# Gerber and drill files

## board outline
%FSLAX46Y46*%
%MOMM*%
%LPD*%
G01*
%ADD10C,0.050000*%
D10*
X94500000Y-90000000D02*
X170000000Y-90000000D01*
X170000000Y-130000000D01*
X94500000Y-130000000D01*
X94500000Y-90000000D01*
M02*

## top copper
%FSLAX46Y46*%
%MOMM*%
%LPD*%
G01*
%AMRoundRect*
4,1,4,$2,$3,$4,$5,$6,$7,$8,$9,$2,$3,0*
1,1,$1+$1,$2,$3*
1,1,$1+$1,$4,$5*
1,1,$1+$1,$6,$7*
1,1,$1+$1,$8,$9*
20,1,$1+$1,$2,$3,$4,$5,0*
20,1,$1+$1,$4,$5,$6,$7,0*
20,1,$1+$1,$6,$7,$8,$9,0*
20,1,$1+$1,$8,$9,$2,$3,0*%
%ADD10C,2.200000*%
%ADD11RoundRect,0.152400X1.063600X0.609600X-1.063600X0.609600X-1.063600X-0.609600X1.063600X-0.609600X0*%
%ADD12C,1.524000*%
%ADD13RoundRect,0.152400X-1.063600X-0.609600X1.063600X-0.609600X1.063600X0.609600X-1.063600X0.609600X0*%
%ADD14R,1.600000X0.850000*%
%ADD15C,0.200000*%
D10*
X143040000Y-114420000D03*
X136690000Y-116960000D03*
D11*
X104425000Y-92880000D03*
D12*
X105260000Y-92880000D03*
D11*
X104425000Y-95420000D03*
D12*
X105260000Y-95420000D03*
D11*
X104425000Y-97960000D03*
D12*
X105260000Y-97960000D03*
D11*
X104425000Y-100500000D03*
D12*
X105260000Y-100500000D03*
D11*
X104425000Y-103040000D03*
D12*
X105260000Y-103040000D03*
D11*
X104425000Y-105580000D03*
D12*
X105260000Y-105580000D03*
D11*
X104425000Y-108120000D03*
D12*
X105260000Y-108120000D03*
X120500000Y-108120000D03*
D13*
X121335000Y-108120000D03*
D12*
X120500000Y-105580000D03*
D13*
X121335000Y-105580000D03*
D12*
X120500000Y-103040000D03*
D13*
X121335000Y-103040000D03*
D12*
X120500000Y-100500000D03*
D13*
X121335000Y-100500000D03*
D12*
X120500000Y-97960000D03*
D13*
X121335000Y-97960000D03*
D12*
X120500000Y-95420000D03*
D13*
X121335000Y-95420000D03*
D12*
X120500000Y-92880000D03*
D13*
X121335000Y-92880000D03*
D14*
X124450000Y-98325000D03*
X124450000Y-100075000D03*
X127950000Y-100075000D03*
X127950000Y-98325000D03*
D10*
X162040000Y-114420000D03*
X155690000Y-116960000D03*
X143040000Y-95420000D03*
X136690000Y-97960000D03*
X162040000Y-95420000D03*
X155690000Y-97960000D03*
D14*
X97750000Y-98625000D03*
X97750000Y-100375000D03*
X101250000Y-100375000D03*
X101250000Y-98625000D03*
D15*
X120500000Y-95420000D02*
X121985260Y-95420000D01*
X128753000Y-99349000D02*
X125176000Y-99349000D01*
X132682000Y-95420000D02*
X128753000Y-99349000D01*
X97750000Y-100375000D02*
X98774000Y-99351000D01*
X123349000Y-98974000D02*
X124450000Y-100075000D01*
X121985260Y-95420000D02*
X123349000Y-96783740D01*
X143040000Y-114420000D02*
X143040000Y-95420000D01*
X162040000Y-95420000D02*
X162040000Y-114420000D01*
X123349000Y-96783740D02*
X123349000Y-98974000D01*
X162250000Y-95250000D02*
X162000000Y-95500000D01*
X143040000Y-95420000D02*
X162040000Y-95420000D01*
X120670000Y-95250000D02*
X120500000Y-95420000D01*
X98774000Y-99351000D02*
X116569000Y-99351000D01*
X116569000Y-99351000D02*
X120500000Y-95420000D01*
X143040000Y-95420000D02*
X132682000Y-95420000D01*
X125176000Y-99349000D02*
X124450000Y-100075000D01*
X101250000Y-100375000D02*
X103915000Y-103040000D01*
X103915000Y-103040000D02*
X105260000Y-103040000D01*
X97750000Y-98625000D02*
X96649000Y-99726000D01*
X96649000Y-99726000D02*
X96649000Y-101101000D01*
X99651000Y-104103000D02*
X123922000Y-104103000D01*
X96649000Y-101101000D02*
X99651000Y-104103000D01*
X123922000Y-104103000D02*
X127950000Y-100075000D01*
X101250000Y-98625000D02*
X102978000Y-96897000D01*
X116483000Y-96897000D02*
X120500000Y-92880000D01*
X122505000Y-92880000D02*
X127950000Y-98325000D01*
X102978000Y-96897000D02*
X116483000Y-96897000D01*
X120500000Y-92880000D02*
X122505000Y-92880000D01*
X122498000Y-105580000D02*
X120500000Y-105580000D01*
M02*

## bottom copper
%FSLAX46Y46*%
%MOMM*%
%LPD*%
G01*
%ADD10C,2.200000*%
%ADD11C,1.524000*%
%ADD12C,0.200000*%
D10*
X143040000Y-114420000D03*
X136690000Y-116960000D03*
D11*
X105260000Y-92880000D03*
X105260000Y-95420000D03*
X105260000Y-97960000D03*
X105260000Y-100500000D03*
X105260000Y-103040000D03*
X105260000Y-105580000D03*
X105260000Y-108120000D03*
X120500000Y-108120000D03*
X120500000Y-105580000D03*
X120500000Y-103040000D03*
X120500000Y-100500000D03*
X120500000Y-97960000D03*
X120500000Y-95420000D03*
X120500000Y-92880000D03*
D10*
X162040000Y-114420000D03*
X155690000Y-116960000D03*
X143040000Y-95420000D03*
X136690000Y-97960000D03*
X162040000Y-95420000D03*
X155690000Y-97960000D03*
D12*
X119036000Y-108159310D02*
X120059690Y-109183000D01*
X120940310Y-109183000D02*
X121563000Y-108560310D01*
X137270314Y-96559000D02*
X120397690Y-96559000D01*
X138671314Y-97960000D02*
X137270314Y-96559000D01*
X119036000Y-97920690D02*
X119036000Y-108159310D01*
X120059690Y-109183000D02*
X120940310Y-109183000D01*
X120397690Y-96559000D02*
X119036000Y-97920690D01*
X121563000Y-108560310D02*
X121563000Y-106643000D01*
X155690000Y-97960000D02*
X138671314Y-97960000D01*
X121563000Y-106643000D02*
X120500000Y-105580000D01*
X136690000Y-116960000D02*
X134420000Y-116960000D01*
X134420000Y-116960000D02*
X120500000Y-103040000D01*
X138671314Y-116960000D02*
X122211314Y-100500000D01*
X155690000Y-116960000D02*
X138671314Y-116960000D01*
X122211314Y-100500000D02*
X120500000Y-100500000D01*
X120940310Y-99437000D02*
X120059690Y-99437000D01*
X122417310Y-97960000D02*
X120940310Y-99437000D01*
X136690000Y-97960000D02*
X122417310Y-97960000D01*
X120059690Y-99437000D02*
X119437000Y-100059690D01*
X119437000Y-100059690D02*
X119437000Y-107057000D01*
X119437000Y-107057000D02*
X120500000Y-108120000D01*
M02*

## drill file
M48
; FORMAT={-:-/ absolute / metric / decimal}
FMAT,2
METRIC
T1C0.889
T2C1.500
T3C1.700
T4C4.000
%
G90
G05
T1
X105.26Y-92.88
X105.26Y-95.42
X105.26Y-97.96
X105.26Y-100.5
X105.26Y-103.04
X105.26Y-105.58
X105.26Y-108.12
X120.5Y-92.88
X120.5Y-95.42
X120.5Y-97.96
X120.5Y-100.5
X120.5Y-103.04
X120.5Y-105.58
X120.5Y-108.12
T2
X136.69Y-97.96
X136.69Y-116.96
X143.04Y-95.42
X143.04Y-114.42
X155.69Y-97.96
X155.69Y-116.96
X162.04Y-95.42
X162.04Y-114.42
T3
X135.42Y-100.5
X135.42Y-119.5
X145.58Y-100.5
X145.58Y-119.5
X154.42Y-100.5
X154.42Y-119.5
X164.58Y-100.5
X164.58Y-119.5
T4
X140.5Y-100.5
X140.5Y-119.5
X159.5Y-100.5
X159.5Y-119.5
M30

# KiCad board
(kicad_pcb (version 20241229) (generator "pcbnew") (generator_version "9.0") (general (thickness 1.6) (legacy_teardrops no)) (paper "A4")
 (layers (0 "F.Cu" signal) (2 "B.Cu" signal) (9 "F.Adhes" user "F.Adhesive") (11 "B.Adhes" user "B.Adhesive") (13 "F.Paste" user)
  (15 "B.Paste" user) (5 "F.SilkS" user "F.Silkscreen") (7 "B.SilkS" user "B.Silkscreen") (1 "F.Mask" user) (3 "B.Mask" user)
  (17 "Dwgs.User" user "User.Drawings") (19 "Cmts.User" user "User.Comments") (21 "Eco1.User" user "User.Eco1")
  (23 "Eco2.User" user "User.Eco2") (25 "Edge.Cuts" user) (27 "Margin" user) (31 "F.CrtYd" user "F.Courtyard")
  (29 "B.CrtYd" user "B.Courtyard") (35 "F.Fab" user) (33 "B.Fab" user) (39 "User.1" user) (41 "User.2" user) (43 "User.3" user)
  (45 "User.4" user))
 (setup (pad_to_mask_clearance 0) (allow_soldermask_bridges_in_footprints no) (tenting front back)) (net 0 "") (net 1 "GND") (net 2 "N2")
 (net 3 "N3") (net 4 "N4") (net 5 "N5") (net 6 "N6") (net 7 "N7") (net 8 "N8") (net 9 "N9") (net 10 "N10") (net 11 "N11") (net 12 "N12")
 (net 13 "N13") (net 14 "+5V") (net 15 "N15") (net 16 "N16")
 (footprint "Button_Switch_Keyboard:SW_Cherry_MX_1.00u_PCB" (layer "F.Cu") (at 143.04 114.42)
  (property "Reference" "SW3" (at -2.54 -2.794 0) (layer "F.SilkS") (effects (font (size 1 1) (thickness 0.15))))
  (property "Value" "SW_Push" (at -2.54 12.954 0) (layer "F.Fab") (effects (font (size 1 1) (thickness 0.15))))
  (pad "" np_thru_hole circle (at -7.62 5.08) (size 1.7 1.7) (drill 1.7) (layers "*.Cu" "*.Mask"))
  (pad "" np_thru_hole circle (at -2.54 5.08) (size 4 4) (drill 4) (layers "*.Cu" "*.Mask"))
  (pad "" np_thru_hole circle (at 2.54 5.08) (size 1.7 1.7) (drill 1.7) (layers "*.Cu" "*.Mask"))
  (pad "1" thru_hole circle (at 0 0) (size 2.2 2.2) (drill 1.5) (layers "*.Cu" "*.Mask") (remove_unused_layers no) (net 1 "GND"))
  (pad "2" thru_hole circle (at -6.35 2.54) (size 2.2 2.2) (drill 1.5) (layers "*.Cu" "*.Mask") (remove_unused_layers no) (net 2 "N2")))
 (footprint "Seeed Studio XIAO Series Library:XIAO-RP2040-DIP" (layer "F.Cu") (at 112.88 100.5)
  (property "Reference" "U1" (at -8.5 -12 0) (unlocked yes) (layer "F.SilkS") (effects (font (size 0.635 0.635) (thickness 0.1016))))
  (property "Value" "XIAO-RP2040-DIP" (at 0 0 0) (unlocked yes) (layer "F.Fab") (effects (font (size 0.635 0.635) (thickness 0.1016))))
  (pad "1" smd roundrect (at -8.455 -7.62 180) (size 2.432 1.524) (layers "F.Cu" "F.Mask") (roundrect_rratio 0.1) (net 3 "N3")
   (thermal_bridge_angle 45))
  (pad "1" thru_hole circle (at -7.62 -7.62 180) (size 1.524 1.524) (drill 0.889) (layers "*.Cu" "*.Mask") (remove_unused_layers no)
   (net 3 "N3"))
  (pad "2" smd roundrect (at -8.455 -5.08 180) (size 2.432 1.524) (layers "F.Cu" "F.Mask") (roundrect_rratio 0.1) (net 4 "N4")
   (thermal_bridge_angle 45))
  (pad "2" thru_hole circle (at -7.62 -5.08 180) (size 1.524 1.524) (drill 0.889) (layers "*.Cu" "*.Mask") (remove_unused_layers no)
   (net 4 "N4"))
  (pad "3" smd roundrect (at -8.455 -2.54 180) (size 2.432 1.524) (layers "F.Cu" "F.Mask") (roundrect_rratio 0.1) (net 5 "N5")
   (thermal_bridge_angle 45))
  (pad "3" thru_hole circle (at -7.62 -2.54 180) (size 1.524 1.524) (drill 0.889) (layers "*.Cu" "*.Mask") (remove_unused_layers no)
   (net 5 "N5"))
  (pad "4" smd roundrect (at -8.455 0 180) (size 2.432 1.524) (layers "F.Cu" "F.Mask") (roundrect_rratio 0.1) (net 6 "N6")
   (thermal_bridge_angle 45))
  (pad "4" thru_hole circle (at -7.62 0 180) (size 1.524 1.524) (drill 0.889) (layers "*.Cu" "*.Mask") (remove_unused_layers no)
   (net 6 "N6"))
  (pad "5" smd roundrect (at -8.455 2.54 180) (size 2.432 1.524) (layers "F.Cu" "F.Mask") (roundrect_rratio 0.1) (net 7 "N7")
   (thermal_bridge_angle 45))
  (pad "5" thru_hole circle (at -7.62 2.54 180) (size 1.524 1.524) (drill 0.889) (layers "*.Cu" "*.Mask") (remove_unused_layers no)
   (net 7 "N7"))
  (pad "6" smd roundrect (at -8.455 5.08 180) (size 2.432 1.524) (layers "F.Cu" "F.Mask") (roundrect_rratio 0.1) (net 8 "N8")
   (thermal_bridge_angle 45))
  (pad "6" thru_hole circle (at -7.62 5.08 180) (size 1.524 1.524) (drill 0.889) (layers "*.Cu" "*.Mask") (remove_unused_layers no)
   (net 8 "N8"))
  (pad "7" smd roundrect (at -8.455 7.62 180) (size 2.432 1.524) (layers "F.Cu" "F.Mask") (roundrect_rratio 0.1) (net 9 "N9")
   (thermal_bridge_angle 45))
  (pad "7" thru_hole circle (at -7.62 7.62 180) (size 1.524 1.524) (drill 0.889) (layers "*.Cu" "*.Mask") (remove_unused_layers no)
   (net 9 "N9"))
  (pad "8" thru_hole circle (at 7.62 7.62) (size 1.524 1.524) (drill 0.889) (layers "*.Cu" "*.Mask") (remove_unused_layers no)
   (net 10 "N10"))
  (pad "8" smd roundrect (at 8.455 7.62) (size 2.432 1.524) (layers "F.Cu" "F.Mask") (roundrect_rratio 0.1) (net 10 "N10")
   (thermal_bridge_angle 45))
  (pad "9" thru_hole circle (at 7.62 5.08) (size 1.524 1.524) (drill 0.889) (layers "*.Cu" "*.Mask") (remove_unused_layers no)
   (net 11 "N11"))
  (pad "9" smd roundrect (at 8.455 5.08) (size 2.432 1.524) (layers "F.Cu" "F.Mask") (roundrect_rratio 0.1) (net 11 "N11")
   (thermal_bridge_angle 45))
  (pad "10" thru_hole circle (at 7.62 2.54) (size 1.524 1.524) (drill 0.889) (layers "*.Cu" "*.Mask") (remove_unused_layers no) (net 2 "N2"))
  (pad "10" smd roundrect (at 8.455 2.54) (size 2.432 1.524) (layers "F.Cu" "F.Mask") (roundrect_rratio 0.1) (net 2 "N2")
   (thermal_bridge_angle 45))
  (pad "11" thru_hole circle (at 7.62 0) (size 1.524 1.524) (drill 0.889) (layers "*.Cu" "*.Mask") (remove_unused_layers no) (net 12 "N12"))
  (pad "11" smd roundrect (at 8.455 0) (size 2.432 1.524) (layers "F.Cu" "F.Mask") (roundrect_rratio 0.1) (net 12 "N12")
   (thermal_bridge_angle 45))
  (pad "12" thru_hole circle (at 7.62 -2.54) (size 1.524 1.524) (drill 0.889) (layers "*.Cu" "*.Mask") (remove_unused_layers no)
   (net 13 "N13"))
  (pad "12" smd roundrect (at 8.455 -2.54) (size 2.432 1.524) (layers "F.Cu" "F.Mask") (roundrect_rratio 0.1) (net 13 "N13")
   (thermal_bridge_angle 45))
  (pad "13" thru_hole circle (at 7.62 -5.08) (size 1.524 1.524) (drill 0.889) (layers "*.Cu" "*.Mask") (remove_unused_layers no)
   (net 1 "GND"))
  (pad "13" smd roundrect (at 8.455 -5.08) (size 2.432 1.524) (layers "F.Cu" "F.Mask") (roundrect_rratio 0.1) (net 1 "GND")
   (thermal_bridge_angle 45))
  (pad "14" thru_hole circle (at 7.62 -7.62) (size 1.524 1.524) (drill 0.889) (layers "*.Cu" "*.Mask") (remove_unused_layers no)
   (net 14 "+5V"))
  (pad "14" smd roundrect (at 8.455 -7.62) (size 2.432 1.524) (layers "F.Cu" "F.Mask") (roundrect_rratio 0.1) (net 14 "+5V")
   (thermal_bridge_angle 45)))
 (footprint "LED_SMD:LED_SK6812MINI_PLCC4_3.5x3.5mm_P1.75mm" (layer "F.Cu") (at 126.2 99.2)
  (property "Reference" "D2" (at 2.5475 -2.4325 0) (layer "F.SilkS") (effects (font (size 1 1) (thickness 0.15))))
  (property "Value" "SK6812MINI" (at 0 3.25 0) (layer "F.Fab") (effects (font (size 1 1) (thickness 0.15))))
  (pad "1" smd rect (at -1.75 -0.875) (size 1.6 0.85) (layers "F.Cu" "F.Mask" "F.Paste") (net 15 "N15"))
  (pad "2" smd rect (at -1.75 0.875) (size 1.6 0.85) (layers "F.Cu" "F.Mask" "F.Paste") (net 1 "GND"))
  (pad "3" smd rect (at 1.75 0.875) (size 1.6 0.85) (layers "F.Cu" "F.Mask" "F.Paste") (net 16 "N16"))
  (pad "4" smd rect (at 1.75 -0.875) (size 1.6 0.85) (layers "F.Cu" "F.Mask" "F.Paste") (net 14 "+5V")))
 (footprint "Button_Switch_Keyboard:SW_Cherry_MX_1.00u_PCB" (layer "F.Cu") (at 162.04 114.42)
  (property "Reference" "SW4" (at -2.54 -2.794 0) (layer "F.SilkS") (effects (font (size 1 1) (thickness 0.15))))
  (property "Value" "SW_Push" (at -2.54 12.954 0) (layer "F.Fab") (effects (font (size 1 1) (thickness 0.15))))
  (pad "" np_thru_hole circle (at -7.62 5.08) (size 1.7 1.7) (drill 1.7) (layers "*.Cu" "*.Mask"))
  (pad "" np_thru_hole circle (at -2.54 5.08) (size 4 4) (drill 4) (layers "*.Cu" "*.Mask"))
  (pad "" np_thru_hole circle (at 2.54 5.08) (size 1.7 1.7) (drill 1.7) (layers "*.Cu" "*.Mask"))
  (pad "1" thru_hole circle (at 0 0) (size 2.2 2.2) (drill 1.5) (layers "*.Cu" "*.Mask") (remove_unused_layers no) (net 1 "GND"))
  (pad "2" thru_hole circle (at -6.35 2.54) (size 2.2 2.2) (drill 1.5) (layers "*.Cu" "*.Mask") (remove_unused_layers no) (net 12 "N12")))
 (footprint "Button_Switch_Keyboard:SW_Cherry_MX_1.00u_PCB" (layer "F.Cu") (at 143.04 95.42)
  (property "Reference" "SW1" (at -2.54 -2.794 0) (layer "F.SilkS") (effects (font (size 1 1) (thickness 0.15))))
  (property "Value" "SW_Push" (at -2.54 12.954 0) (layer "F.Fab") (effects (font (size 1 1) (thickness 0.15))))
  (pad "" np_thru_hole circle (at -7.62 5.08) (size 1.7 1.7) (drill 1.7) (layers "*.Cu" "*.Mask"))
  (pad "" np_thru_hole circle (at -2.54 5.08) (size 4 4) (drill 4) (layers "*.Cu" "*.Mask"))
  (pad "" np_thru_hole circle (at 2.54 5.08) (size 1.7 1.7) (drill 1.7) (layers "*.Cu" "*.Mask"))
  (pad "1" thru_hole circle (at 0 0) (size 2.2 2.2) (drill 1.5) (layers "*.Cu" "*.Mask") (remove_unused_layers no) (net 1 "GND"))
  (pad "2" thru_hole circle (at -6.35 2.54) (size 2.2 2.2) (drill 1.5) (layers "*.Cu" "*.Mask") (remove_unused_layers no) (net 10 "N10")))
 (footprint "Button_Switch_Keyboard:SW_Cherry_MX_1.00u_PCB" (layer "F.Cu") (at 162.04 95.42)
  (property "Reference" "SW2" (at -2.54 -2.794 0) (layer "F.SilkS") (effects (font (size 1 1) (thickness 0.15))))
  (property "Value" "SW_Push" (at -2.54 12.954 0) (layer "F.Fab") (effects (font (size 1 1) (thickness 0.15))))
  (pad "" np_thru_hole circle (at -7.62 5.08) (size 1.7 1.7) (drill 1.7) (layers "*.Cu" "*.Mask"))
  (pad "" np_thru_hole circle (at -2.54 5.08) (size 4 4) (drill 4) (layers "*.Cu" "*.Mask"))
  (pad "" np_thru_hole circle (at 2.54 5.08) (size 1.7 1.7) (drill 1.7) (layers "*.Cu" "*.Mask"))
  (pad "1" thru_hole circle (at 0 0) (size 2.2 2.2) (drill 1.5) (layers "*.Cu" "*.Mask") (remove_unused_layers no) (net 1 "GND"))
  (pad "2" thru_hole circle (at -6.35 2.54) (size 2.2 2.2) (drill 1.5) (layers "*.Cu" "*.Mask") (remove_unused_layers no) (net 11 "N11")))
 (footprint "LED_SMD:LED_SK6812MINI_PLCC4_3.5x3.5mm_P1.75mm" (layer "F.Cu") (at 99.5 99.5)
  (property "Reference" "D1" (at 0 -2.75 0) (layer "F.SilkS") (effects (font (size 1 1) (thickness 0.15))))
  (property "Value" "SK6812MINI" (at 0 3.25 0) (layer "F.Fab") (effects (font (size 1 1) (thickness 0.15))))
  (pad "1" smd rect (at -1.75 -0.875) (size 1.6 0.85) (layers "F.Cu" "F.Mask" "F.Paste") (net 16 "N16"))
  (pad "2" smd rect (at -1.75 0.875) (size 1.6 0.85) (layers "F.Cu" "F.Mask" "F.Paste") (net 1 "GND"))
  (pad "3" smd rect (at 1.75 0.875) (size 1.6 0.85) (layers "F.Cu" "F.Mask" "F.Paste") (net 7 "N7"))
  (pad "4" smd rect (at 1.75 -0.875) (size 1.6 0.85) (layers "F.Cu" "F.Mask" "F.Paste") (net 14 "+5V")))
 (gr_rect (start 94.5 90) (end 170 130) (stroke (width 0.05) (type default)) (fill no) (layer "Edge.Cuts"))
 (segment (start 120.5 95.42) (end 121.98526 95.42) (width 0.2) (layer "F.Cu") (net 1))
 (segment (start 128.753 99.349) (end 125.176 99.349) (width 0.2) (layer "F.Cu") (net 1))
 (segment (start 132.682 95.42) (end 128.753 99.349) (width 0.2) (layer "F.Cu") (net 1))
 (segment (start 97.75 100.375) (end 98.774 99.351) (width 0.2) (layer "F.Cu") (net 1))
 (segment (start 123.349 98.974) (end 124.45 100.075) (width 0.2) (layer "F.Cu") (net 1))
 (segment (start 121.98526 95.42) (end 123.349 96.78374) (width 0.2) (layer "F.Cu") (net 1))
 (segment (start 143.04 114.42) (end 143.04 95.42) (width 0.2) (layer "F.Cu") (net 1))
 (segment (start 162.04 95.42) (end 162.04 114.42) (width 0.2) (layer "F.Cu") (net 1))
 (segment (start 123.349 96.78374) (end 123.349 98.974) (width 0.2) (layer "F.Cu") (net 1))
 (segment (start 162.25 95.25) (end 162 95.5) (width 0.2) (layer "F.Cu") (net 1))
 (segment (start 143.04 95.42) (end 162.04 95.42) (width 0.2) (layer "F.Cu") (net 1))
 (segment (start 120.67 95.25) (end 120.5 95.42) (width 0.2) (layer "F.Cu") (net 1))
 (segment (start 98.774 99.351) (end 116.569 99.351) (width 0.2) (layer "F.Cu") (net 1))
 (segment (start 116.569 99.351) (end 120.5 95.42) (width 0.2) (layer "F.Cu") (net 1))
 (segment (start 143.04 95.42) (end 132.682 95.42) (width 0.2) (layer "F.Cu") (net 1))
 (segment (start 125.176 99.349) (end 124.45 100.075) (width 0.2) (layer "F.Cu") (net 1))
 (segment (start 101.25 100.375) (end 103.915 103.04) (width 0.2) (layer "F.Cu") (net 7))
 (segment (start 103.915 103.04) (end 105.26 103.04) (width 0.2) (layer "F.Cu") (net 7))
 (segment (start 97.75 98.625) (end 96.649 99.726) (width 0.2) (layer "F.Cu") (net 16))
 (segment (start 96.649 99.726) (end 96.649 101.101) (width 0.2) (layer "F.Cu") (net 16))
 (segment (start 99.651 104.103) (end 123.922 104.103) (width 0.2) (layer "F.Cu") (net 16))
 (segment (start 96.649 101.101) (end 99.651 104.103) (width 0.2) (layer "F.Cu") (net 16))
 (segment (start 123.922 104.103) (end 127.95 100.075) (width 0.2) (layer "F.Cu") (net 16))
 (segment (start 101.25 98.625) (end 102.978 96.897) (width 0.2) (layer "F.Cu") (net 14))
 (segment (start 116.483 96.897) (end 120.5 92.88) (width 0.2) (layer "F.Cu") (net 14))
 (segment (start 122.505 92.88) (end 127.95 98.325) (width 0.2) (layer "F.Cu") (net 14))
 (segment (start 102.978 96.897) (end 116.483 96.897) (width 0.2) (layer "F.Cu") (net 14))
 (segment (start 120.5 92.88) (end 122.505 92.88) (width 0.2) (layer "F.Cu") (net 14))
 (segment (start 122.498 105.58) (end 120.5 105.58) (width 0.2) (layer "F.Cu") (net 11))
 (segment (start 119.036 108.15931) (end 120.05969 109.183) (width 0.2) (layer "B.Cu") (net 11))
 (segment (start 120.94031 109.183) (end 121.563 108.56031) (width 0.2) (layer "B.Cu") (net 11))
 (segment (start 137.270314 96.559) (end 120.39769 96.559) (width 0.2) (layer "B.Cu") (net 11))
 (segment (start 138.671314 97.96) (end 137.270314 96.559) (width 0.2) (layer "B.Cu") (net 11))
 (segment (start 119.036 97.92069) (end 119.036 108.15931) (width 0.2) (layer "B.Cu") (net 11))
 (segment (start 120.05969 109.183) (end 120.94031 109.183) (width 0.2) (layer "B.Cu") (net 11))
 (segment (start 120.39769 96.559) (end 119.036 97.92069) (width 0.2) (layer "B.Cu") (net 11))
 (segment (start 121.563 108.56031) (end 121.563 106.643) (width 0.2) (layer "B.Cu") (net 11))
 (segment (start 155.69 97.96) (end 138.671314 97.96) (width 0.2) (layer "B.Cu") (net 11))
 (segment (start 121.563 106.643) (end 120.5 105.58) (width 0.2) (layer "B.Cu") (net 11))
 (segment (start 136.69 116.96) (end 134.42 116.96) (width 0.2) (layer "B.Cu") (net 2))
 (segment (start 134.42 116.96) (end 120.5 103.04) (width 0.2) (layer "B.Cu") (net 2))
 (segment (start 138.671314 116.96) (end 122.211314 100.5) (width 0.2) (layer "B.Cu") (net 12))
 (segment (start 155.69 116.96) (end 138.671314 116.96) (width 0.2) (layer "B.Cu") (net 12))
 (segment (start 122.211314 100.5) (end 120.5 100.5) (width 0.2) (layer "B.Cu") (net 12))
 (segment (start 120.94031 99.437) (end 120.05969 99.437) (width 0.2) (layer "B.Cu") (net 10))
 (segment (start 122.41731 97.96) (end 120.94031 99.437) (width 0.2) (layer "B.Cu") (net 10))
 (segment (start 136.69 97.96) (end 122.41731 97.96) (width 0.2) (layer "B.Cu") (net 10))
 (segment (start 120.05969 99.437) (end 119.437 100.05969) (width 0.2) (layer "B.Cu") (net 10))
 (segment (start 119.437 100.05969) (end 119.437 107.057) (width 0.2) (layer "B.Cu") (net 10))
 (segment (start 119.437 107.057) (end 120.5 108.12) (width 0.2) (layer "B.Cu") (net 10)))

